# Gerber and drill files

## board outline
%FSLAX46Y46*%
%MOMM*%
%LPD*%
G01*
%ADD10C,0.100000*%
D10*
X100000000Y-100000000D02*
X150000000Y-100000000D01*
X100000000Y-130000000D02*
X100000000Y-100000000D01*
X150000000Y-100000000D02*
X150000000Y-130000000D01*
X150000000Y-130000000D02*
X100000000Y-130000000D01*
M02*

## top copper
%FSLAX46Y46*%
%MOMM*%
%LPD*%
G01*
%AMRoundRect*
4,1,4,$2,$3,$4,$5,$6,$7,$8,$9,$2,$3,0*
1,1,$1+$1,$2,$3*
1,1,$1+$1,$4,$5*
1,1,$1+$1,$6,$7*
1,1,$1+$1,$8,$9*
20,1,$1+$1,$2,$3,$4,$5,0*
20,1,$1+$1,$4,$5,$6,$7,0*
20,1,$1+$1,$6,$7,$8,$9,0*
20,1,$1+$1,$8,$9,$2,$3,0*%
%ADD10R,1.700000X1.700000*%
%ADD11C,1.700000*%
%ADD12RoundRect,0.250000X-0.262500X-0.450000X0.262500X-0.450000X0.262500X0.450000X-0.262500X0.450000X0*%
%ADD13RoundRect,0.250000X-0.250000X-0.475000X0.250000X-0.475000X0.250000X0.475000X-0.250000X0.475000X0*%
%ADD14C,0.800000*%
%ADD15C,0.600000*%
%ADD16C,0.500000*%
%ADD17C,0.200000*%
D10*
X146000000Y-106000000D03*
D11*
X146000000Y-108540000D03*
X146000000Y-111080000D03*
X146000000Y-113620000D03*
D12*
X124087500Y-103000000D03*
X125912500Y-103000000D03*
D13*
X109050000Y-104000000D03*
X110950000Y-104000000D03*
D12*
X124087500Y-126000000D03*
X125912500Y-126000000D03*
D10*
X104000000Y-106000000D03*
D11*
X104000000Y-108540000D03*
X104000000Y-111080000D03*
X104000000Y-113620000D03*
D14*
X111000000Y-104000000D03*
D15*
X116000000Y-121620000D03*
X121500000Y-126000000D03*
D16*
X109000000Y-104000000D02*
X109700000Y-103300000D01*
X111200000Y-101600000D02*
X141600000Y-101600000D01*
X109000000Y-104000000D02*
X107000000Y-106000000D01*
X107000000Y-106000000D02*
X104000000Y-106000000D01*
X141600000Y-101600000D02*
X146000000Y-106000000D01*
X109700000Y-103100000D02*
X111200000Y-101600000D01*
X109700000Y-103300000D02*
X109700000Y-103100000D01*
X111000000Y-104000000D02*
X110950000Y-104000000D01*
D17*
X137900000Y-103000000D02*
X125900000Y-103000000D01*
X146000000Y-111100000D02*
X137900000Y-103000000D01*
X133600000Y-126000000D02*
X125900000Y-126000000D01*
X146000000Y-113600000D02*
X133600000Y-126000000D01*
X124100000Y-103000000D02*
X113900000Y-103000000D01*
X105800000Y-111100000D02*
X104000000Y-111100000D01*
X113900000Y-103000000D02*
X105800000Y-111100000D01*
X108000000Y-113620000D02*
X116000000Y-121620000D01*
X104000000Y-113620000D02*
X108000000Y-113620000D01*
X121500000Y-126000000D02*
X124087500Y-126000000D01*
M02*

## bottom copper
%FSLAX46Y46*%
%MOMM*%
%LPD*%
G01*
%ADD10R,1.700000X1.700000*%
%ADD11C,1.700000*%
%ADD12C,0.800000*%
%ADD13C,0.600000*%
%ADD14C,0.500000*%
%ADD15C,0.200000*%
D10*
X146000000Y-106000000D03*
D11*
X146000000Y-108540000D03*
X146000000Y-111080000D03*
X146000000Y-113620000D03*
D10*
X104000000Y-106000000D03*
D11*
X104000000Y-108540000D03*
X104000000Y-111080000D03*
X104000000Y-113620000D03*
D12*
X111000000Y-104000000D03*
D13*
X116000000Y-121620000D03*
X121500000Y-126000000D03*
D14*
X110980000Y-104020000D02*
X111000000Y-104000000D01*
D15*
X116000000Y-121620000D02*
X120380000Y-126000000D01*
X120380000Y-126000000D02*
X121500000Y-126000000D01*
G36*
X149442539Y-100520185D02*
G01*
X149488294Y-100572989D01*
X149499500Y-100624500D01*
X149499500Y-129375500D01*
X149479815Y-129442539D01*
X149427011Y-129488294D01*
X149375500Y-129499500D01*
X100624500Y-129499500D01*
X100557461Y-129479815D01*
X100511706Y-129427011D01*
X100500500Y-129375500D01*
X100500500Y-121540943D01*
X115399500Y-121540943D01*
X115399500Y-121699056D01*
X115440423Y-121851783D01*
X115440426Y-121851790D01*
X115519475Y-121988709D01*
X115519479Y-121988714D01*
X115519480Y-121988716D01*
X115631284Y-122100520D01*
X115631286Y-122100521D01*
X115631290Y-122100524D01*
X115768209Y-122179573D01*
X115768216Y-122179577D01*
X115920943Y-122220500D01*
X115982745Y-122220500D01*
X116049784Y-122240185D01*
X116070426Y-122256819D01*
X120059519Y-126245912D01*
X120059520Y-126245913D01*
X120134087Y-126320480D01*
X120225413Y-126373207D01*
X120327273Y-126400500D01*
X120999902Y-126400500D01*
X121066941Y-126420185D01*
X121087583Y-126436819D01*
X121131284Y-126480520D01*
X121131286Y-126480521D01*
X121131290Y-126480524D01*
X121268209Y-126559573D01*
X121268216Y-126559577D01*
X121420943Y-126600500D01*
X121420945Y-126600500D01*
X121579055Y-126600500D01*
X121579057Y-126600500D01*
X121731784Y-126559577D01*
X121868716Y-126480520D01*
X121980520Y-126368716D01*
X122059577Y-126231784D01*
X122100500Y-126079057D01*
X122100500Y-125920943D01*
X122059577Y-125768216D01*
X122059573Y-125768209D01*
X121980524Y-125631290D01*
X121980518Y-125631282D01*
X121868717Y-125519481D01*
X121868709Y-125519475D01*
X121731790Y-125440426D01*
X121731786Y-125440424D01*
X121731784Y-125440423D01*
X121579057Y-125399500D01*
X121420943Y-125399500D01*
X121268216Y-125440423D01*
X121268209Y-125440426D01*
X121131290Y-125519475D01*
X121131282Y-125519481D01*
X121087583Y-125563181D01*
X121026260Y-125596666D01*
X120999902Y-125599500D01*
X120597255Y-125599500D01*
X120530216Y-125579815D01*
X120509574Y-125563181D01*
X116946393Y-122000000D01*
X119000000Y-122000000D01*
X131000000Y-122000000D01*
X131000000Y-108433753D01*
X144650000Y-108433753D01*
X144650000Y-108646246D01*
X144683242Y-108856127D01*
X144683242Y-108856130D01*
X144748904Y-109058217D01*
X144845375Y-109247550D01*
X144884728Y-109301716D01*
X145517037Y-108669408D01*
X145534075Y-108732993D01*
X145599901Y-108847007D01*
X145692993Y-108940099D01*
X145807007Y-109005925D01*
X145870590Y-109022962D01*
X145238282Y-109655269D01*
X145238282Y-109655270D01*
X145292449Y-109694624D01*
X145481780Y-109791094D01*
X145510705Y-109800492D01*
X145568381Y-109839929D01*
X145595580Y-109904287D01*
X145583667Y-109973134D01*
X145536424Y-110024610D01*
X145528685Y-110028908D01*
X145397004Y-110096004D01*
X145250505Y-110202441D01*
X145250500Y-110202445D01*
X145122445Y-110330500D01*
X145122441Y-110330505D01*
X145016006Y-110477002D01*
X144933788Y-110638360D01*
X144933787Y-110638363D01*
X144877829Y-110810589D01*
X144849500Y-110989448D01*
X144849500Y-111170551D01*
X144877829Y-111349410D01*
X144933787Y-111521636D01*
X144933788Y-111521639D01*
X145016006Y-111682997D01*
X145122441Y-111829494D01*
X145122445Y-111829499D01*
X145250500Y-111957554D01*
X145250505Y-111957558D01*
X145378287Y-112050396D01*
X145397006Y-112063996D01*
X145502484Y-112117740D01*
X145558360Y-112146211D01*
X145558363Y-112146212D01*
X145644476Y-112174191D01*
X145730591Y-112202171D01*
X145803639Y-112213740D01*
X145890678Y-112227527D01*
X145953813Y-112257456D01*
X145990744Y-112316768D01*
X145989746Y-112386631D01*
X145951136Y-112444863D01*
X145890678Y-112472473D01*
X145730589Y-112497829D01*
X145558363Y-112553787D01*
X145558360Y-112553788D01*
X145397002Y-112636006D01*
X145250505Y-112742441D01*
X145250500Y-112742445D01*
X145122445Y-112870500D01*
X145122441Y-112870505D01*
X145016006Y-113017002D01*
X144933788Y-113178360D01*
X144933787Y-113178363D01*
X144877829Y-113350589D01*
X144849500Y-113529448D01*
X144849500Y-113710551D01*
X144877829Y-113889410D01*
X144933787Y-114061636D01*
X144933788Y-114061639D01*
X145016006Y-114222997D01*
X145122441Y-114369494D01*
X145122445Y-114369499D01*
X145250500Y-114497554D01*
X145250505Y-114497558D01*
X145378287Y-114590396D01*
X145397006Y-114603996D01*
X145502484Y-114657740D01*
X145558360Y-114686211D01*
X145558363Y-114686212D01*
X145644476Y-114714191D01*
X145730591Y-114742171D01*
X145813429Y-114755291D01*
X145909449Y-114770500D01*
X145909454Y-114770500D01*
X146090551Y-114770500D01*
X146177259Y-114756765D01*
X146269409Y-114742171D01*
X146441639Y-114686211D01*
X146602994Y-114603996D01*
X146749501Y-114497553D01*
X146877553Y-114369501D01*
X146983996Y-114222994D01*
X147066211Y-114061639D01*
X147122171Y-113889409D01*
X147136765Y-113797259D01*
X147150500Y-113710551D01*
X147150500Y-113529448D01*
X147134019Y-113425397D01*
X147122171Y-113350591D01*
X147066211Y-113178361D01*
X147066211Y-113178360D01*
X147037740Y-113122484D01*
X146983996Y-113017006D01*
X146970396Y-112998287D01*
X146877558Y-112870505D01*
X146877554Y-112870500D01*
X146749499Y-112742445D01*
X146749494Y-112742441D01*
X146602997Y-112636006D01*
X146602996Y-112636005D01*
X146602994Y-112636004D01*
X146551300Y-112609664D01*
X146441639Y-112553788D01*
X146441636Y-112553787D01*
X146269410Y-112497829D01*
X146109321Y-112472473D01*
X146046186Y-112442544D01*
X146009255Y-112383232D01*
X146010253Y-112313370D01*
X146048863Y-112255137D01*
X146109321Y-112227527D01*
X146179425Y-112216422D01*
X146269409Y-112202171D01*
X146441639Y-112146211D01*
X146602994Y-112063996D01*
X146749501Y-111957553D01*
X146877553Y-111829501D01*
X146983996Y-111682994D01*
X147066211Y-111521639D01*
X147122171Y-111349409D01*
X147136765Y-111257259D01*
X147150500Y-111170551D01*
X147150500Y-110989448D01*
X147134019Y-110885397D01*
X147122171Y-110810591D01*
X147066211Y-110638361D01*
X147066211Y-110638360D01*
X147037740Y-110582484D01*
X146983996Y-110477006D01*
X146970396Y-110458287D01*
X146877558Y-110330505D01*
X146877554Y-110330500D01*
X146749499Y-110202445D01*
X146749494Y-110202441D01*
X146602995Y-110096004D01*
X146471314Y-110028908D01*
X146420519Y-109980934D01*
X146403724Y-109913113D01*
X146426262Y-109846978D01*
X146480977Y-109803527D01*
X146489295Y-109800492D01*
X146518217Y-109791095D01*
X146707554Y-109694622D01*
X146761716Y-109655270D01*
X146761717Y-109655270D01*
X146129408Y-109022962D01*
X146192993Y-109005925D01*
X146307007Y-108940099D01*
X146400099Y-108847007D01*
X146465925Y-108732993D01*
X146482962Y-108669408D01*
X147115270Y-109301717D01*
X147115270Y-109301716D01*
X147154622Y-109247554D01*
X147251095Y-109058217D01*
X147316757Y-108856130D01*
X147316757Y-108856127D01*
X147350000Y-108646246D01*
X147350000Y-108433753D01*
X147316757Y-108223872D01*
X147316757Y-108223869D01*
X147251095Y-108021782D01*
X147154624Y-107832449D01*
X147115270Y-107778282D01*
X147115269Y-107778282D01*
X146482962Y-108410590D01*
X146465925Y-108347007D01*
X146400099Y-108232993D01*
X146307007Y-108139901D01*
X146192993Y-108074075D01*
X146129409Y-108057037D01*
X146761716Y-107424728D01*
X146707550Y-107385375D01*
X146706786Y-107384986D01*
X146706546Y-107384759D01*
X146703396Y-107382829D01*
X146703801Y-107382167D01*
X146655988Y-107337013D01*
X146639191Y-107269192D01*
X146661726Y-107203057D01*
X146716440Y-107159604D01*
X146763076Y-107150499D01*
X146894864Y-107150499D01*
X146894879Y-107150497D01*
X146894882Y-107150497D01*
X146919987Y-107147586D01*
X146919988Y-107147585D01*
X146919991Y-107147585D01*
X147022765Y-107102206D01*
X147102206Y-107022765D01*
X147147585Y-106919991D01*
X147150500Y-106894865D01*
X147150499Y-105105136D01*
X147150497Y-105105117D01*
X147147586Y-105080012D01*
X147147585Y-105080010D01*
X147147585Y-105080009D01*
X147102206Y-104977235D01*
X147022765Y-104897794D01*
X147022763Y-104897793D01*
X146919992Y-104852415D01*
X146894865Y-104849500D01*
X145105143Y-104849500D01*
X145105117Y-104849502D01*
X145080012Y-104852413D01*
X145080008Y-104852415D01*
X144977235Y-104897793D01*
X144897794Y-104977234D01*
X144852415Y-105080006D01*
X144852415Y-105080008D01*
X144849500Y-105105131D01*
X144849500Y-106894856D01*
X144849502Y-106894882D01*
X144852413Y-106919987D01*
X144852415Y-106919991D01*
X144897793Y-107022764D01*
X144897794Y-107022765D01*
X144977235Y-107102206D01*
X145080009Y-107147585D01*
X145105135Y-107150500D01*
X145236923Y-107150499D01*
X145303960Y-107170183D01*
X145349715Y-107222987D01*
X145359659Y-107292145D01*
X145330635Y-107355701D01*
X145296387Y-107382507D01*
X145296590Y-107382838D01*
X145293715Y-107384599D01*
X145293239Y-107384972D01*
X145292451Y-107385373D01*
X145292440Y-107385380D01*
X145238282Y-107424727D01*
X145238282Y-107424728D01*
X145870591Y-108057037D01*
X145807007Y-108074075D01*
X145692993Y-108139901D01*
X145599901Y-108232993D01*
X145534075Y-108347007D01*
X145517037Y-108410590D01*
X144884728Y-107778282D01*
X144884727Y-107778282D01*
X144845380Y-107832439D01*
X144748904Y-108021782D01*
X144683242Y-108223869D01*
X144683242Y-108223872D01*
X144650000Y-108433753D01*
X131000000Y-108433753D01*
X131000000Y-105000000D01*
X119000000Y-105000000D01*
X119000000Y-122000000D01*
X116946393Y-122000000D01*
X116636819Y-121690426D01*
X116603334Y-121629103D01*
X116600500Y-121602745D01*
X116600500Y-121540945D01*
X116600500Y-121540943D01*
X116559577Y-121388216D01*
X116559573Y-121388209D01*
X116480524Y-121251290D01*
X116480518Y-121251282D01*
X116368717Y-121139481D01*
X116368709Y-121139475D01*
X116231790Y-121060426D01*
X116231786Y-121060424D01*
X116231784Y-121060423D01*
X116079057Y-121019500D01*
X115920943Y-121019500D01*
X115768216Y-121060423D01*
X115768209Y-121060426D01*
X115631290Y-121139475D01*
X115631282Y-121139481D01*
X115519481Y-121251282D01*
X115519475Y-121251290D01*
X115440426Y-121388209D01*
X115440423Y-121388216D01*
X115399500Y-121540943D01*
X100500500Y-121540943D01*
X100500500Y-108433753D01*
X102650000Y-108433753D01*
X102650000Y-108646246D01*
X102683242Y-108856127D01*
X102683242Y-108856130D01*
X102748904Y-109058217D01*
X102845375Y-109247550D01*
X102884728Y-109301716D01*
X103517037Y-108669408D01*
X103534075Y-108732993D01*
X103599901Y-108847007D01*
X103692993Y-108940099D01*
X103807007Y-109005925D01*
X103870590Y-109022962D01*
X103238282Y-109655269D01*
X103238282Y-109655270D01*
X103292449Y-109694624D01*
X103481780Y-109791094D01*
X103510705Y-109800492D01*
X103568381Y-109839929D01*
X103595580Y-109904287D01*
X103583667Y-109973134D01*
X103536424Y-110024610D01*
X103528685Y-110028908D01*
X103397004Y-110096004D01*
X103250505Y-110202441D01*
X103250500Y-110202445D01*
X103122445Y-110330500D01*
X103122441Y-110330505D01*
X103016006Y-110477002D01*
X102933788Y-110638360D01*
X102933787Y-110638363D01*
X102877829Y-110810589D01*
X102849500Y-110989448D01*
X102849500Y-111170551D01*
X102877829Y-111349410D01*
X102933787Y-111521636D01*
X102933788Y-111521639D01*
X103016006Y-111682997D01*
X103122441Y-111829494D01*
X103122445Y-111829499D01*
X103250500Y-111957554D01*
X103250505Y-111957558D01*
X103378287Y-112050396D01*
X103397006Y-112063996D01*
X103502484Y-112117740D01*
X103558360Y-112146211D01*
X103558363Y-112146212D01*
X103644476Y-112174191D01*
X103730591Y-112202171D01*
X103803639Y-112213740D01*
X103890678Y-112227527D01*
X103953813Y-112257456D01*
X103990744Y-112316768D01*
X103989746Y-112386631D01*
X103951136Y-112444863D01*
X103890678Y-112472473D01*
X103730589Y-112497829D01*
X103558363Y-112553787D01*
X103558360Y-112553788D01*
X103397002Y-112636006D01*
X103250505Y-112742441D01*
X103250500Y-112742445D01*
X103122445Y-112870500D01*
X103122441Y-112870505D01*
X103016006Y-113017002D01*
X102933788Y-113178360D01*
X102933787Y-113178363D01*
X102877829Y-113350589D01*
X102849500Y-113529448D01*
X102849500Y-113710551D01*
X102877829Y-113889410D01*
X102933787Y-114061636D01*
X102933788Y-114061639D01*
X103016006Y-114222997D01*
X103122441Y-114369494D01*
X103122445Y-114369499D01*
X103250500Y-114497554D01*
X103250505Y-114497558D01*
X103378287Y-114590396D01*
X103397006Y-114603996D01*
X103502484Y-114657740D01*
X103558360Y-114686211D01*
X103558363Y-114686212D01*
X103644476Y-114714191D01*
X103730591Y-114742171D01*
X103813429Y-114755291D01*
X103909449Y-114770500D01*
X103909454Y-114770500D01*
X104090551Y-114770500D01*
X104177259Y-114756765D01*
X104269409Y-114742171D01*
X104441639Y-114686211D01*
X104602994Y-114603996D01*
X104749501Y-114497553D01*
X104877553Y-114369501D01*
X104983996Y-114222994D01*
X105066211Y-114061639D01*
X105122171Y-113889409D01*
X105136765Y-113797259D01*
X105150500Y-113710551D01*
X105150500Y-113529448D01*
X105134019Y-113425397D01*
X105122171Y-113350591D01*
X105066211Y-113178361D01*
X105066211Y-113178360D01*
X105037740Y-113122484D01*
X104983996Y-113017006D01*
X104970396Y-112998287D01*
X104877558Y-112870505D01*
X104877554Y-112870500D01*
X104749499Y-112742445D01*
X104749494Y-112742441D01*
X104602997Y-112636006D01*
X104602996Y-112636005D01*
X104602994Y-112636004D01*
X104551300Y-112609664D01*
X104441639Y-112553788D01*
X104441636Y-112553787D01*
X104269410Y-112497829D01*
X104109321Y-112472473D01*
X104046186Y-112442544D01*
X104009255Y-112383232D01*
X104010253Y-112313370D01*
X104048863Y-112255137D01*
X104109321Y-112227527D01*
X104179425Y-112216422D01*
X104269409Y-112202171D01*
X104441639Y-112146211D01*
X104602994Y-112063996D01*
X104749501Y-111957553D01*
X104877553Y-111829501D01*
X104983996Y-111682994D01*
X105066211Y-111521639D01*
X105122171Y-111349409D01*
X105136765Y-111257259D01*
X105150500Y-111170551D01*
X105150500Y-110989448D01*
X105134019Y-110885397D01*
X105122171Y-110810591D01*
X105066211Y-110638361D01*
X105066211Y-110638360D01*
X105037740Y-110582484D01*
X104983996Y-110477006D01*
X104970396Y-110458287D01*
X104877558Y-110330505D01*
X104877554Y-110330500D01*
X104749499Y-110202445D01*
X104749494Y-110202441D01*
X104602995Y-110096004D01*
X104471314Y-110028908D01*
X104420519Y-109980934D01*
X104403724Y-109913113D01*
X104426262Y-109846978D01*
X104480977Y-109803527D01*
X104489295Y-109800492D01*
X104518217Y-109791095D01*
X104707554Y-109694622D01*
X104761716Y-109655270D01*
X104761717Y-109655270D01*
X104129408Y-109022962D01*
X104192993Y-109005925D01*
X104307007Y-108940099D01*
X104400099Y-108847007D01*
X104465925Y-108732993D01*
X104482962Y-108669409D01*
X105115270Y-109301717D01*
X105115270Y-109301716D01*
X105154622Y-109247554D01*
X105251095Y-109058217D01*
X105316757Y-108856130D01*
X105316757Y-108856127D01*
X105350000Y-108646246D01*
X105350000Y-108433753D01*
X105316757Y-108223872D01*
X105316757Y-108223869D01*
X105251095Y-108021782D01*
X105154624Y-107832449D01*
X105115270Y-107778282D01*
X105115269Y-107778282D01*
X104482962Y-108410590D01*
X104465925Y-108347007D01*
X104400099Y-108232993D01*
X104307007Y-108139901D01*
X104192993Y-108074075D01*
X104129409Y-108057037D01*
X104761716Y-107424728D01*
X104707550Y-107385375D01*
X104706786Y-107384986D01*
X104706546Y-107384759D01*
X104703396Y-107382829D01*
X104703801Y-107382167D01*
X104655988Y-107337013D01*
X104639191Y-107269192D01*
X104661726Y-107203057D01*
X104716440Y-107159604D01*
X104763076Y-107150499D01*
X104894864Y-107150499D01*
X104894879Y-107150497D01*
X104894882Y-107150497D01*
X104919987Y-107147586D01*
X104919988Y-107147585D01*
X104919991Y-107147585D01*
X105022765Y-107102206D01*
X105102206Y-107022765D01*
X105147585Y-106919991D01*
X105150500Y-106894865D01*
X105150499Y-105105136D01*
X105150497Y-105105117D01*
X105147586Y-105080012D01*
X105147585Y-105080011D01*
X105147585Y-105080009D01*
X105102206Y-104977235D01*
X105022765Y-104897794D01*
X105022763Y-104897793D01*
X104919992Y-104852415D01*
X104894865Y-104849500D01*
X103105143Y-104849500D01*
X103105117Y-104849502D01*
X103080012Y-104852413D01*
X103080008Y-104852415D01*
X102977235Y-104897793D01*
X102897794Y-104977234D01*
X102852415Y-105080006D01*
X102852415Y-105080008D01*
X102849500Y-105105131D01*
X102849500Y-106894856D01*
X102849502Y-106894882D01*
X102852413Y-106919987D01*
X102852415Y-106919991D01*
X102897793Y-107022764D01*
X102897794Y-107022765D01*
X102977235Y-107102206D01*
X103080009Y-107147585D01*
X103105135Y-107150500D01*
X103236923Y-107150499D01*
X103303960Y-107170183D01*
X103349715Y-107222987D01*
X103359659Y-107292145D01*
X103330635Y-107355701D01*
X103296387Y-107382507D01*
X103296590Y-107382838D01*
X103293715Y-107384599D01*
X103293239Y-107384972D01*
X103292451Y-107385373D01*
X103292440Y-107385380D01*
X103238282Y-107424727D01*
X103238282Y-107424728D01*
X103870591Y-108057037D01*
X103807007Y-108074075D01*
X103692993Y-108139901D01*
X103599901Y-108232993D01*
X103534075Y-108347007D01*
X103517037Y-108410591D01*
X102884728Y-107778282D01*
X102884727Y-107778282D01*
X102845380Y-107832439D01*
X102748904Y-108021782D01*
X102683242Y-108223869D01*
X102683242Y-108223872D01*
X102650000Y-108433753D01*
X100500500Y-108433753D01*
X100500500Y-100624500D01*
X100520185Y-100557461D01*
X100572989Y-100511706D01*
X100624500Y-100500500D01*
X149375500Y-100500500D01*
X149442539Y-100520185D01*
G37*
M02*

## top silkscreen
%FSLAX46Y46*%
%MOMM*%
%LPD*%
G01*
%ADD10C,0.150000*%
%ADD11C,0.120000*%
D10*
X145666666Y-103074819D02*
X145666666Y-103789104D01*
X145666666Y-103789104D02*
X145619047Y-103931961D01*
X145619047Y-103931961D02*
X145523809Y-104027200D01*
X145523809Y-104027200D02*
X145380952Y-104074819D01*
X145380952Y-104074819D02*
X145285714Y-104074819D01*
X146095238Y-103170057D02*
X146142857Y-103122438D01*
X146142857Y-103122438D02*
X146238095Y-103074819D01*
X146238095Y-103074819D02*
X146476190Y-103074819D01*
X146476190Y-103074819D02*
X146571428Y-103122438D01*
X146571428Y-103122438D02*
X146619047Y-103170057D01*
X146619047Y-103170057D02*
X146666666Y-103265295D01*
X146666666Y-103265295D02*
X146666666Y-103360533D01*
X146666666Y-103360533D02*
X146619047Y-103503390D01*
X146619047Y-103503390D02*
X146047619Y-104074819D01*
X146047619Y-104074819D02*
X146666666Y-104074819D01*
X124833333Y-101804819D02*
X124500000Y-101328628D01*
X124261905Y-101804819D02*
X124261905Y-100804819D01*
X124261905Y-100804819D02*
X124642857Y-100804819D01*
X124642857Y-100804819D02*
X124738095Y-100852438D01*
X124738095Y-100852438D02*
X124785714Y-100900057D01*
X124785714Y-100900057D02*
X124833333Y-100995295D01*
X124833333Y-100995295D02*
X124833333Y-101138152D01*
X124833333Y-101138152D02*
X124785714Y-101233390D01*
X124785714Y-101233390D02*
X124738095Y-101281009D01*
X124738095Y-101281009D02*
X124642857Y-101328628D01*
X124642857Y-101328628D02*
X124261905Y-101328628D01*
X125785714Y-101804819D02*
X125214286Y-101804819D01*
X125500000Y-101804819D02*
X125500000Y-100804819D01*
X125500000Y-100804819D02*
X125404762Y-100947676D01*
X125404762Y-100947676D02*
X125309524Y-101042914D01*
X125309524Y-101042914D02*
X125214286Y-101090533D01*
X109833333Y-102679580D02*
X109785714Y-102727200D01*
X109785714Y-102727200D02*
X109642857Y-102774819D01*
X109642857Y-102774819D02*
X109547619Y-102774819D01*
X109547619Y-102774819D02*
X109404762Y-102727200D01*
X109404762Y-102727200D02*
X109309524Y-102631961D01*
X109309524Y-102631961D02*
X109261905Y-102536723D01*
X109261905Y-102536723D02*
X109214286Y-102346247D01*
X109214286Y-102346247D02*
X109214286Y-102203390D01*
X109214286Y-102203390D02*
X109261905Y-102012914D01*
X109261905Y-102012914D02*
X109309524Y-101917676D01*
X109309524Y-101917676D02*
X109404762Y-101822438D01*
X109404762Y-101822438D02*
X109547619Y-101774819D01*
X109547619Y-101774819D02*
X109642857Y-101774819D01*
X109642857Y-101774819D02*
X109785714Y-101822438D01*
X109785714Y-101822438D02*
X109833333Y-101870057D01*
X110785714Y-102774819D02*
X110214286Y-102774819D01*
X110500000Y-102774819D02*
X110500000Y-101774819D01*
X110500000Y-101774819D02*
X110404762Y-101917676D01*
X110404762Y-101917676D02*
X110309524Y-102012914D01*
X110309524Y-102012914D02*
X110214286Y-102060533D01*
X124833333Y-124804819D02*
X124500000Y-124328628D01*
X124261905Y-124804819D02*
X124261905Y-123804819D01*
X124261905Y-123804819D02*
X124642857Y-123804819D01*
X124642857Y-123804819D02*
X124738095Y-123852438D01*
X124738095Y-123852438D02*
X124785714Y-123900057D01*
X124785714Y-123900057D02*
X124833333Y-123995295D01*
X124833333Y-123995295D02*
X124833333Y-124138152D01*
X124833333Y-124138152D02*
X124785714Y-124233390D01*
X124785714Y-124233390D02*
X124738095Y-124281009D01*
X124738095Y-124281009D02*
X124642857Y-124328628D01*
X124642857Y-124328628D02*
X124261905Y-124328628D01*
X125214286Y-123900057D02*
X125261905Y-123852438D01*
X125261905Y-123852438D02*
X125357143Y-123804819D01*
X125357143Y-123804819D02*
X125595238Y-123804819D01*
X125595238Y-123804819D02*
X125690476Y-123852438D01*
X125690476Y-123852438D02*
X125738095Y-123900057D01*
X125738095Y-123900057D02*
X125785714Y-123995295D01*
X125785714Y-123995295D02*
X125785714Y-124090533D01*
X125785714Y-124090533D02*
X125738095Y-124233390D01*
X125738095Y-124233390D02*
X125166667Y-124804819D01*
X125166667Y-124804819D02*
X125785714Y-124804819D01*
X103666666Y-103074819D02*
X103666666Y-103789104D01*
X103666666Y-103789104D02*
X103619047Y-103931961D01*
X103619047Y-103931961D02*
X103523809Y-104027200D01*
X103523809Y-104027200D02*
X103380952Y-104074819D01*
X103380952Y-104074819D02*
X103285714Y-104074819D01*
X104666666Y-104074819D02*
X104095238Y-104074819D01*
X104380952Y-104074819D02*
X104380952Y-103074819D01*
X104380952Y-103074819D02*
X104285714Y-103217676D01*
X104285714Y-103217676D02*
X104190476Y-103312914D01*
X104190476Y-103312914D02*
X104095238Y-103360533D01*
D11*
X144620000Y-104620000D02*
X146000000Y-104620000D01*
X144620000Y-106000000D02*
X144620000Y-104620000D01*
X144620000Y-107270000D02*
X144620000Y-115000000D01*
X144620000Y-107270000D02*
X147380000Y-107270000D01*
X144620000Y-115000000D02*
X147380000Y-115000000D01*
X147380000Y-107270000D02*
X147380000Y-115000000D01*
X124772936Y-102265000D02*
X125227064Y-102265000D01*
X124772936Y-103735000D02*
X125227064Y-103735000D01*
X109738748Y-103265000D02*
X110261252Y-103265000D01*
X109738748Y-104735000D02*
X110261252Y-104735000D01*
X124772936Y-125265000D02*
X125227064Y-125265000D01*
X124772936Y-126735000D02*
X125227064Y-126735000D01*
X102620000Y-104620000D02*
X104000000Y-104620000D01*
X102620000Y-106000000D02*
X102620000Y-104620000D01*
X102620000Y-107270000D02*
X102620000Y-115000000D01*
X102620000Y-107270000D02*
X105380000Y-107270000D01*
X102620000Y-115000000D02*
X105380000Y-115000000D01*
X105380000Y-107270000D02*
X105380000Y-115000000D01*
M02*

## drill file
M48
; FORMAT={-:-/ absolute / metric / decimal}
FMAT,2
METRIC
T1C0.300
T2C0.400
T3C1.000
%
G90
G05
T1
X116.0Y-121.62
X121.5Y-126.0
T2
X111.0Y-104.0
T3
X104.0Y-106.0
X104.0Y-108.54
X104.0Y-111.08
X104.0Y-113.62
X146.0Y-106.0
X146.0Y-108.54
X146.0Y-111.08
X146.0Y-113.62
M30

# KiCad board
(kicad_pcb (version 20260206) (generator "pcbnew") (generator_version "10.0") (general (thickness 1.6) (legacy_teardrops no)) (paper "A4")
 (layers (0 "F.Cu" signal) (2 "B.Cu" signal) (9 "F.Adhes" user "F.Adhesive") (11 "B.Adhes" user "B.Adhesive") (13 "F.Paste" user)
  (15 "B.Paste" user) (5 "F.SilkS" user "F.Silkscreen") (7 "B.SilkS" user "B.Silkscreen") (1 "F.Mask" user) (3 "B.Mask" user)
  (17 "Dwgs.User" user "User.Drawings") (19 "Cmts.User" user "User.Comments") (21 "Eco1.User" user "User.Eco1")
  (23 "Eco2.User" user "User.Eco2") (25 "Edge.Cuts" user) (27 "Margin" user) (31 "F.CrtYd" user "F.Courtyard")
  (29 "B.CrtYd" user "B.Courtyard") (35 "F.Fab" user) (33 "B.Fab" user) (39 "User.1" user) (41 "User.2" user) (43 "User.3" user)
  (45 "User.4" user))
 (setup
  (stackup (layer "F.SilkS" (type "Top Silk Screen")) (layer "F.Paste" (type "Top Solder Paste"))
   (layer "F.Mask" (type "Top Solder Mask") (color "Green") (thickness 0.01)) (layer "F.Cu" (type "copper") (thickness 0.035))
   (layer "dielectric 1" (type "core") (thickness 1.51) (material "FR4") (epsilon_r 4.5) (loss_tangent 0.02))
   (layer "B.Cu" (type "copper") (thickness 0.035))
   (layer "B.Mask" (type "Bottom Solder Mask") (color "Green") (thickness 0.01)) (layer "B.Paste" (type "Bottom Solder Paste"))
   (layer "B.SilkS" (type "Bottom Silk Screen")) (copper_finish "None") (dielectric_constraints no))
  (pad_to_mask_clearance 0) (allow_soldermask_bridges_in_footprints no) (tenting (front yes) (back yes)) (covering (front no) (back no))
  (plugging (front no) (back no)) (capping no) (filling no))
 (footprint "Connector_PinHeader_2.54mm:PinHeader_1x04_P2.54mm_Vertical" (layer "F.Cu") (at 146 106)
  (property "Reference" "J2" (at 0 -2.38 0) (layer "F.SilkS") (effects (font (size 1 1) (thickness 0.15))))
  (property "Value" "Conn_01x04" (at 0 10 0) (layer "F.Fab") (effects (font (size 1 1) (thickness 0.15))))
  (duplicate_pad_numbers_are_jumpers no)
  (fp_line (start -1.38 -1.38) (end 0 -1.38) (stroke (width 0.12) (type solid)) (layer "F.SilkS"))
  (fp_line (start -1.38 0) (end -1.38 -1.38) (stroke (width 0.12) (type solid)) (layer "F.SilkS"))
  (fp_line (start -1.38 1.27) (end -1.38 9) (stroke (width 0.12) (type solid)) (layer "F.SilkS"))
  (fp_line (start -1.38 1.27) (end 1.38 1.27) (stroke (width 0.12) (type solid)) (layer "F.SilkS"))
  (fp_line (start -1.38 9) (end 1.38 9) (stroke (width 0.12) (type solid)) (layer "F.SilkS"))
  (fp_line (start 1.38 1.27) (end 1.38 9) (stroke (width 0.12) (type solid)) (layer "F.SilkS"))
  (pad "1" thru_hole rect (at 0 0) (size 1.7 1.7) (drill 1) (layers "*.Cu" "*.Mask") (remove_unused_layers no) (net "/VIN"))
  (pad "2" thru_hole circle (at 0 2.54) (size 1.7 1.7) (drill 1) (layers "*.Cu" "*.Mask") (remove_unused_layers no) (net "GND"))
  (pad "3" thru_hole circle (at 0 5.08) (size 1.7 1.7) (drill 1) (layers "*.Cu" "*.Mask") (remove_unused_layers no) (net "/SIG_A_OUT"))
  (pad "4" thru_hole circle (at 0 7.62) (size 1.7 1.7) (drill 1) (layers "*.Cu" "*.Mask") (remove_unused_layers no) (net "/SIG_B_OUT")))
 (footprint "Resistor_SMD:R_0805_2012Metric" (layer "F.Cu") (at 125 103)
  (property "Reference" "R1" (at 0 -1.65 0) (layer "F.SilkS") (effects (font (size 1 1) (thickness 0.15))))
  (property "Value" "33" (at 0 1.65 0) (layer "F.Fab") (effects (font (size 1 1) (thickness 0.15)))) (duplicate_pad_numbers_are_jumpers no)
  (fp_line (start -0.227064 -0.735) (end 0.227064 -0.735) (stroke (width 0.12) (type solid)) (layer "F.SilkS"))
  (fp_line (start -0.227064 0.735) (end 0.227064 0.735) (stroke (width 0.12) (type solid)) (layer "F.SilkS"))
  (pad "1" smd roundrect (at -0.9125 0) (size 1.025 1.4) (layers "F.Cu" "F.Mask" "F.Paste") (roundrect_rratio 0.243902) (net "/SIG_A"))
  (pad "2" smd roundrect (at 0.9125 0) (size 1.025 1.4) (layers "F.Cu" "F.Mask" "F.Paste") (roundrect_rratio 0.243902) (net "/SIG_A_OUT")))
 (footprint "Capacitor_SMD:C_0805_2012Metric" (layer "F.Cu") (at 110 104)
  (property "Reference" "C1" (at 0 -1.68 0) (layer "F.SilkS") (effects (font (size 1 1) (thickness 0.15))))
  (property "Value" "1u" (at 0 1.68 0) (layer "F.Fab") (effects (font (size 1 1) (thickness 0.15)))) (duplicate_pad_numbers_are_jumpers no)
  (fp_line (start -0.261252 -0.735) (end 0.261252 -0.735) (stroke (width 0.12) (type solid)) (layer "F.SilkS"))
  (fp_line (start -0.261252 0.735) (end 0.261252 0.735) (stroke (width 0.12) (type solid)) (layer "F.SilkS"))
  (pad "1" smd roundrect (at -0.95 0) (size 1 1.45) (layers "F.Cu" "F.Mask" "F.Paste") (roundrect_rratio 0.25) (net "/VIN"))
  (pad "2" smd roundrect (at 0.95 0) (size 1 1.45) (layers "F.Cu" "F.Mask" "F.Paste") (roundrect_rratio 0.25) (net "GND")))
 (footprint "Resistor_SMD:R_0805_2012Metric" (layer "F.Cu") (at 125 126)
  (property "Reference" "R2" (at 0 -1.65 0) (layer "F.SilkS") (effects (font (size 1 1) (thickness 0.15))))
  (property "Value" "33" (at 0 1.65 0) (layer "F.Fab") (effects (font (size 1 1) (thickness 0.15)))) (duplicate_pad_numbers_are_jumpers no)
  (fp_line (start -0.227064 -0.735) (end 0.227064 -0.735) (stroke (width 0.12) (type solid)) (layer "F.SilkS"))
  (fp_line (start -0.227064 0.735) (end 0.227064 0.735) (stroke (width 0.12) (type solid)) (layer "F.SilkS"))
  (pad "1" smd roundrect (at -0.9125 0) (size 1.025 1.4) (layers "F.Cu" "F.Mask" "F.Paste") (roundrect_rratio 0.243902) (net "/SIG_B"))
  (pad "2" smd roundrect (at 0.9125 0) (size 1.025 1.4) (layers "F.Cu" "F.Mask" "F.Paste") (roundrect_rratio 0.243902) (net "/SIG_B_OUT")))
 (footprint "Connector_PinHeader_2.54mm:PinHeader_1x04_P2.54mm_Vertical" (layer "F.Cu") (at 104 106)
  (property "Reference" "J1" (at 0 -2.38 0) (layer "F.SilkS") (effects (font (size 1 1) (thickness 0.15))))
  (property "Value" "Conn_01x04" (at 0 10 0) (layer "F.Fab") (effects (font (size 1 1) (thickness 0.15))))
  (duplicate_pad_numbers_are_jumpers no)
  (fp_line (start -1.38 -1.38) (end 0 -1.38) (stroke (width 0.12) (type solid)) (layer "F.SilkS"))
  (fp_line (start -1.38 0) (end -1.38 -1.38) (stroke (width 0.12) (type solid)) (layer "F.SilkS"))
  (fp_line (start -1.38 1.27) (end -1.38 9) (stroke (width 0.12) (type solid)) (layer "F.SilkS"))
  (fp_line (start -1.38 1.27) (end 1.38 1.27) (stroke (width 0.12) (type solid)) (layer "F.SilkS"))
  (fp_line (start -1.38 9) (end 1.38 9) (stroke (width 0.12) (type solid)) (layer "F.SilkS"))
  (fp_line (start 1.38 1.27) (end 1.38 9) (stroke (width 0.12) (type solid)) (layer "F.SilkS"))
  (pad "1" thru_hole rect (at 0 0) (size 1.7 1.7) (drill 1) (layers "*.Cu" "*.Mask") (remove_unused_layers no) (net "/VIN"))
  (pad "2" thru_hole circle (at 0 2.54) (size 1.7 1.7) (drill 1) (layers "*.Cu" "*.Mask") (remove_unused_layers no) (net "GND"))
  (pad "3" thru_hole circle (at 0 5.08) (size 1.7 1.7) (drill 1) (layers "*.Cu" "*.Mask") (remove_unused_layers no) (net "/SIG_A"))
  (pad "4" thru_hole circle (at 0 7.62) (size 1.7 1.7) (drill 1) (layers "*.Cu" "*.Mask") (remove_unused_layers no) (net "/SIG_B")))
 (gr_line (start 100 100) (end 150 100) (stroke (width 0.1) (type default)) (layer "Edge.Cuts"))
 (gr_line (start 100 130) (end 100 100) (stroke (width 0.1) (type default)) (layer "Edge.Cuts"))
 (gr_line (start 150 100) (end 150 130) (stroke (width 0.1) (type default)) (layer "Edge.Cuts"))
 (gr_line (start 150 130) (end 100 130) (stroke (width 0.1) (type default)) (layer "Edge.Cuts"))
 (segment (start 109 104) (end 109.7 103.3) (width 0.5) (layer "F.Cu") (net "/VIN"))
 (segment (start 111.2 101.6) (end 141.6 101.6) (width 0.5) (layer "F.Cu") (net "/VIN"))
 (segment (start 109 104) (end 107 106) (width 0.5) (layer "F.Cu") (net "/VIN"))
 (segment (start 107 106) (end 104 106) (width 0.5) (layer "F.Cu") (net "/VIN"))
 (segment (start 141.6 101.6) (end 146 106) (width 0.5) (layer "F.Cu") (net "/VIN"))
 (segment (start 109.7 103.1) (end 111.2 101.6) (width 0.5) (layer "F.Cu") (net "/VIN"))
 (segment (start 109.7 103.3) (end 109.7 103.1) (width 0.5) (layer "F.Cu") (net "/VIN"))
 (segment (start 111 104) (end 110.95 104) (width 0.5) (layer "F.Cu") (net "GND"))
 (via (at 111 104) (size 0.8) (drill 0.4) (layers "F.Cu" "B.Cu") (capping yes) (filling yes) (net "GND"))
 (segment (start 110.98 104.02) (end 111 104) (width 0.5) (layer "B.Cu") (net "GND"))
 (segment (start 137.9 103) (end 125.9 103) (width 0.2) (layer "F.Cu") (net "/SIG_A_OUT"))
 (segment (start 146 111.1) (end 137.9 103) (width 0.2) (layer "F.Cu") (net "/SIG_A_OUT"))
 (segment (start 133.6 126) (end 125.9 126) (width 0.2) (layer "F.Cu") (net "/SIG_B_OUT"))
 (segment (start 146 113.6) (end 133.6 126) (width 0.2) (layer "F.Cu") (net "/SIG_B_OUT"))
 (segment (start 124.1 103) (end 113.9 103) (width 0.2) (layer "F.Cu") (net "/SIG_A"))
 (segment (start 105.8 111.1) (end 104 111.1) (width 0.2) (layer "F.Cu") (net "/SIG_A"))
 (segment (start 113.9 103) (end 105.8 111.1) (width 0.2) (layer "F.Cu") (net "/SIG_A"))
 (segment (start 108 113.62) (end 116 121.62) (width 0.2) (locked yes) (layer "F.Cu") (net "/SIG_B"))
 (segment (start 104 113.62) (end 108 113.62) (width 0.2) (locked yes) (layer "F.Cu") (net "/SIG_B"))
 (segment (start 121.5 126) (end 124.0875 126) (width 0.2) (locked yes) (layer "F.Cu") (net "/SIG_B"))
 (via (at 116 121.62) (size 0.6) (drill 0.3) (layers "F.Cu" "B.Cu") (locked yes) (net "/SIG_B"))
 (via (at 121.5 126) (size 0.6) (drill 0.3) (layers "F.Cu" "B.Cu") (locked yes) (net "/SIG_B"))
 (segment (start 116 121.62) (end 120.38 126) (width 0.2) (locked yes) (layer "B.Cu") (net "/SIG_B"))
 (segment (start 120.38 126) (end 121.5 126) (width 0.2) (locked yes) (layer "B.Cu") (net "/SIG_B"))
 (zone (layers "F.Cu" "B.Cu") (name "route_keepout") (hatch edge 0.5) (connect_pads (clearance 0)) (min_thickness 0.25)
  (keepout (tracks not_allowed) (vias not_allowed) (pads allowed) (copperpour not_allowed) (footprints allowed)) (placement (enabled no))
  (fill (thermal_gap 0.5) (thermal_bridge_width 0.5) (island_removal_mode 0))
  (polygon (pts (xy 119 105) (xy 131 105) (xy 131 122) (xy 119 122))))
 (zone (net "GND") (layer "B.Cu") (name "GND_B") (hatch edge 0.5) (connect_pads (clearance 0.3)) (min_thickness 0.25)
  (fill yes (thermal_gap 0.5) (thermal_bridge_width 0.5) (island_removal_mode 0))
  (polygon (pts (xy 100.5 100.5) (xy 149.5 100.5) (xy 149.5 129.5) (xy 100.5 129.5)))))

